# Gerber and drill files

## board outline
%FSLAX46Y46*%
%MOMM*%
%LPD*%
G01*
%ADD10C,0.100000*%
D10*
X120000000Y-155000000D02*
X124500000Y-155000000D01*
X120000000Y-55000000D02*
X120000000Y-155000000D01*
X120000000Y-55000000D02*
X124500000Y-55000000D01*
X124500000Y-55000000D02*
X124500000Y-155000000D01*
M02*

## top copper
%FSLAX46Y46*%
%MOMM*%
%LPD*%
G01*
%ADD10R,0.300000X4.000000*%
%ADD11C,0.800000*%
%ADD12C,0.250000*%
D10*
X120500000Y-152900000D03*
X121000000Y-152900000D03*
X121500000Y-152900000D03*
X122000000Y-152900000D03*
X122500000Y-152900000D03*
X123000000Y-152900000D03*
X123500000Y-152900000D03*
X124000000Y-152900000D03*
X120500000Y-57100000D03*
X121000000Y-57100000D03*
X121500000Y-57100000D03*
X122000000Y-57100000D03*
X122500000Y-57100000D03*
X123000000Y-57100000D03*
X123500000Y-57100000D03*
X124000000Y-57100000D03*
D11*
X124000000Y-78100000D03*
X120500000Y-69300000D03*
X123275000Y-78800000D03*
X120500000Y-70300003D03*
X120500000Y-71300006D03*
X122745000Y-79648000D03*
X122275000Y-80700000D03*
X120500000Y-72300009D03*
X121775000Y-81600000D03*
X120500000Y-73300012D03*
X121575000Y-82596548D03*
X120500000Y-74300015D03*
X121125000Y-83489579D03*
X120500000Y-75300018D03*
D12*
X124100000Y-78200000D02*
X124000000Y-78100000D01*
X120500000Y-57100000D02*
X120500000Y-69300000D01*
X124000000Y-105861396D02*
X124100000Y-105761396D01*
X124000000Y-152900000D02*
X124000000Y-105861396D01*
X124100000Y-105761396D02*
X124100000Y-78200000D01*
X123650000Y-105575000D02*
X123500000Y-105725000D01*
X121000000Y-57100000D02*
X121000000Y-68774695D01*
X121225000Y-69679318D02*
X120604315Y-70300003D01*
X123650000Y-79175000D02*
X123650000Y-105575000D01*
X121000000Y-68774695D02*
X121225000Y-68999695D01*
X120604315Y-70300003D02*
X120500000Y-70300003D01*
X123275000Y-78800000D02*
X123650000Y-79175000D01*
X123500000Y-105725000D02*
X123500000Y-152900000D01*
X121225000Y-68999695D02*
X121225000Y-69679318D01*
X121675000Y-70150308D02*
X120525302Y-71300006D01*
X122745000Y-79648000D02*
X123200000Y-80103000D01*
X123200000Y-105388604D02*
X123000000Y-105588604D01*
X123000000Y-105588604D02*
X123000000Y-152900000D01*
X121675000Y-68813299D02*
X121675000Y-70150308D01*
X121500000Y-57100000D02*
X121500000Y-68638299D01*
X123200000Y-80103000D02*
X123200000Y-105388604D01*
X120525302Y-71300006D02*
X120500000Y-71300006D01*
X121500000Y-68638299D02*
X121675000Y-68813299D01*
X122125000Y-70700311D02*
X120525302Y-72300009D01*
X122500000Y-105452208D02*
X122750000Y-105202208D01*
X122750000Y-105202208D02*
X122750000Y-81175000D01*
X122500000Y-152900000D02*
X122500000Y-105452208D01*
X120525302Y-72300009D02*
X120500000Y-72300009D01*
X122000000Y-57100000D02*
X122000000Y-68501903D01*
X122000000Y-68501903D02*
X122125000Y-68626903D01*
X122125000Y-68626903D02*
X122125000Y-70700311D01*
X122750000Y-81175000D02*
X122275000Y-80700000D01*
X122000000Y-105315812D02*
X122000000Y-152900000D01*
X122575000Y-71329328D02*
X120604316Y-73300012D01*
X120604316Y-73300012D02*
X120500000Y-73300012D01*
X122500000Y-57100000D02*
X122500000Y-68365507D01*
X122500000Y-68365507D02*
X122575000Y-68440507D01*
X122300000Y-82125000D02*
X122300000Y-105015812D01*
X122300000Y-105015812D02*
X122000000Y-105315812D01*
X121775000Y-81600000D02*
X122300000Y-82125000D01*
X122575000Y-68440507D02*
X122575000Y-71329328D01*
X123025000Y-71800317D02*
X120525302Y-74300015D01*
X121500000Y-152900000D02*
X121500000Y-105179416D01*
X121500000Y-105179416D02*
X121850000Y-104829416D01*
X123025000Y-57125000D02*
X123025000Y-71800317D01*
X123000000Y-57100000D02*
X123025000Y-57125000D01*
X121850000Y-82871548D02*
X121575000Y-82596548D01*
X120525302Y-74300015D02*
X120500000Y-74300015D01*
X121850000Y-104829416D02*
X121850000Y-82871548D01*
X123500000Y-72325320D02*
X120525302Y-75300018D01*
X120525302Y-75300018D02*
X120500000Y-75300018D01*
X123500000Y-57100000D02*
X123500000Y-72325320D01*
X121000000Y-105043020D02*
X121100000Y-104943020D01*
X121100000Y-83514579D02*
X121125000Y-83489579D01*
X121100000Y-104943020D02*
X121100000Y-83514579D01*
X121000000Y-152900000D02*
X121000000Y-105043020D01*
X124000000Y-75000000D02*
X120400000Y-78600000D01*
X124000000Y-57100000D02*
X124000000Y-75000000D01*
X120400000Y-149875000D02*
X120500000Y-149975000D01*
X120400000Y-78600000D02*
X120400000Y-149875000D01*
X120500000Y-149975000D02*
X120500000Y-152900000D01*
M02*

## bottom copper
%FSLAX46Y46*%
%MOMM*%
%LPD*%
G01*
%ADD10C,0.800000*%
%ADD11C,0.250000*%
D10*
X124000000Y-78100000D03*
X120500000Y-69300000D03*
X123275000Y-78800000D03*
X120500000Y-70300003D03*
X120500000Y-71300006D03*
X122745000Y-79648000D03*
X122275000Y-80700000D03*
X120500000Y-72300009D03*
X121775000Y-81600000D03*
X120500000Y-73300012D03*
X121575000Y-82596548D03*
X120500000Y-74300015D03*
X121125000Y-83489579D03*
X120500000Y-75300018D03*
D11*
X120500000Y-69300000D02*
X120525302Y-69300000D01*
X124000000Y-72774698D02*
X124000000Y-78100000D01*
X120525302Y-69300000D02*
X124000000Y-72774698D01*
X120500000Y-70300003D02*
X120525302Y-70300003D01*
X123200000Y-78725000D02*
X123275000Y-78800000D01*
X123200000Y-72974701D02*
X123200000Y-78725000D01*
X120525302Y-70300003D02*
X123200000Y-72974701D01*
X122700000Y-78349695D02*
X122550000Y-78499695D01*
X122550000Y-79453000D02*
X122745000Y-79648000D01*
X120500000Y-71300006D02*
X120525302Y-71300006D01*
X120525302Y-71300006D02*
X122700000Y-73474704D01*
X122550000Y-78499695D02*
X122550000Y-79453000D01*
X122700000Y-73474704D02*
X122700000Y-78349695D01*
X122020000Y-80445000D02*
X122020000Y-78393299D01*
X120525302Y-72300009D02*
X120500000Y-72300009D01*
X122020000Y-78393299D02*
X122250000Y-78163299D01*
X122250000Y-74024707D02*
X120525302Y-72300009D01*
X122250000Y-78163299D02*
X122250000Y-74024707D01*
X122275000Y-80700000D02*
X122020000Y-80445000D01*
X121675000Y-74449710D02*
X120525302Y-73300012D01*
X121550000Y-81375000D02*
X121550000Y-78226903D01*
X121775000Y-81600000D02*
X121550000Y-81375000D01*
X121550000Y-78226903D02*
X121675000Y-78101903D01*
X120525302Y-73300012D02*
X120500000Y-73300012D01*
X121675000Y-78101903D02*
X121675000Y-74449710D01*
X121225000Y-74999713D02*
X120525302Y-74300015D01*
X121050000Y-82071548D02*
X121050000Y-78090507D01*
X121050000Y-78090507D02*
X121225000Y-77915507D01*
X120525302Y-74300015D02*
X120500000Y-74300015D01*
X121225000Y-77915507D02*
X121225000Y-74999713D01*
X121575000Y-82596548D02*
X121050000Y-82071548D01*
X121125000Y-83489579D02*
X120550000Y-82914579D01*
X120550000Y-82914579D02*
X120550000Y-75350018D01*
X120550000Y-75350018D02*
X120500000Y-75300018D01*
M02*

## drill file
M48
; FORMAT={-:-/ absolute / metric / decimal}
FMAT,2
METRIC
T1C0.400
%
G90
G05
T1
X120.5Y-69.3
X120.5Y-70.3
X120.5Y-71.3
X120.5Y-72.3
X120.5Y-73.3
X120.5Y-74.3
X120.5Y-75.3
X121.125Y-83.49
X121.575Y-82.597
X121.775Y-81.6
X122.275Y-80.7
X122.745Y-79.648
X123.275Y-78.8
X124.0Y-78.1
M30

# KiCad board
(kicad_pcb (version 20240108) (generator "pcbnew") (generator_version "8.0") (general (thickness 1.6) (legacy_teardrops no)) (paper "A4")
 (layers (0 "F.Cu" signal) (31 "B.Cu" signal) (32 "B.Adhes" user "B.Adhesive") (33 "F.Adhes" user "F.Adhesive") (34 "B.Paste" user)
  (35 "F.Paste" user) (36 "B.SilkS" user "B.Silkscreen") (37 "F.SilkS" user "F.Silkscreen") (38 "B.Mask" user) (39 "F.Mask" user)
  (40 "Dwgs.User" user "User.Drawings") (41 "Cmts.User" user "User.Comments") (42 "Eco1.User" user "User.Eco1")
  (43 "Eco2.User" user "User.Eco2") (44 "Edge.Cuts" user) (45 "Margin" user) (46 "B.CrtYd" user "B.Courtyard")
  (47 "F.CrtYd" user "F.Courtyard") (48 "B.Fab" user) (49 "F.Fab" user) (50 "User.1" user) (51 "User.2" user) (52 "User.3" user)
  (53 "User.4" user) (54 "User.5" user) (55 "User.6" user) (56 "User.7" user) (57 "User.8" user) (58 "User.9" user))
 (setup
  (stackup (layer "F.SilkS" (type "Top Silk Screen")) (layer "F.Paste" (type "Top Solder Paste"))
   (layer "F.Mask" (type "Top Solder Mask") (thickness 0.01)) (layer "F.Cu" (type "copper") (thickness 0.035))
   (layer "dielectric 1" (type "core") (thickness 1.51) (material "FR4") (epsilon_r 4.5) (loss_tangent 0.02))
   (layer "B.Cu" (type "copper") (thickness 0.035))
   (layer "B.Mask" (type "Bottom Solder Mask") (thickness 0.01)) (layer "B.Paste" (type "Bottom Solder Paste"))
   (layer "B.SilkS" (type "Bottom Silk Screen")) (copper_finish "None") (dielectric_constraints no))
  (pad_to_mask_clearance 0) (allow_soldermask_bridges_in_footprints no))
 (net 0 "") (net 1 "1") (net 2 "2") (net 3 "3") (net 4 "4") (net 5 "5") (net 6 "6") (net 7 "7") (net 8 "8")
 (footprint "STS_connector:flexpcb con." (layer "F.Cu") (at 120 154.9)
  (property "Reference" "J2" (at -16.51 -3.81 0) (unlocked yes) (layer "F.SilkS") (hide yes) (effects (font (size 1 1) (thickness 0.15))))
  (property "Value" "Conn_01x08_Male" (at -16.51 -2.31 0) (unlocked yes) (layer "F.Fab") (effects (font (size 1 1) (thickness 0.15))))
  (pad "1" smd rect (at 0.5 -2) (size 0.3 4) (layers "F.Cu" "F.Paste" "F.Mask") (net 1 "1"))
  (pad "2" smd rect (at 1 -2) (size 0.3 4) (layers "F.Cu" "F.Paste" "F.Mask") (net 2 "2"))
  (pad "3" smd rect (at 1.5 -2) (size 0.3 4) (layers "F.Cu" "F.Paste" "F.Mask") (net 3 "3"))
  (pad "4" smd rect (at 2 -2) (size 0.3 4) (layers "F.Cu" "F.Paste" "F.Mask") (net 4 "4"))
  (pad "5" smd rect (at 2.5 -2) (size 0.3 4) (layers "F.Cu" "F.Paste" "F.Mask") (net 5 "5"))
  (pad "6" smd rect (at 3 -2) (size 0.3 4) (layers "F.Cu" "F.Paste" "F.Mask") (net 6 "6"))
  (pad "7" smd rect (at 3.5 -2) (size 0.3 4) (layers "F.Cu" "F.Paste" "F.Mask") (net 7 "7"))
  (pad "8" smd rect (at 4 -2) (size 0.3 4) (layers "F.Cu" "F.Paste" "F.Mask") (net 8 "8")))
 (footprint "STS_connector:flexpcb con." (layer "F.Cu") (at 120 59.1)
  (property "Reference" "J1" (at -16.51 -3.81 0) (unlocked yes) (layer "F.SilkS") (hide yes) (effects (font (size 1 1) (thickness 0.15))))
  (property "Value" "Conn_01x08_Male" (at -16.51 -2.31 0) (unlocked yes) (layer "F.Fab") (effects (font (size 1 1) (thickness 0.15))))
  (pad "1" smd rect (at 0.5 -2) (size 0.3 4) (layers "F.Cu" "F.Paste" "F.Mask") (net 8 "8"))
  (pad "2" smd rect (at 1 -2) (size 0.3 4) (layers "F.Cu" "F.Paste" "F.Mask") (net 7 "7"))
  (pad "3" smd rect (at 1.5 -2) (size 0.3 4) (layers "F.Cu" "F.Paste" "F.Mask") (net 6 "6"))
  (pad "4" smd rect (at 2 -2) (size 0.3 4) (layers "F.Cu" "F.Paste" "F.Mask") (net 5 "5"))
  (pad "5" smd rect (at 2.5 -2) (size 0.3 4) (layers "F.Cu" "F.Paste" "F.Mask") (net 4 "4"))
  (pad "6" smd rect (at 3 -2) (size 0.3 4) (layers "F.Cu" "F.Paste" "F.Mask") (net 3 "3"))
  (pad "7" smd rect (at 3.5 -2) (size 0.3 4) (layers "F.Cu" "F.Paste" "F.Mask") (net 2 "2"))
  (pad "8" smd rect (at 4 -2) (size 0.3 4) (layers "F.Cu" "F.Paste" "F.Mask") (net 1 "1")))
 (gr_line (start 120 155) (end 124.5 155) (stroke (width 0.1) (type solid)) (layer "Edge.Cuts"))
 (gr_line (start 120 55) (end 120 155) (stroke (width 0.1) (type solid)) (layer "Edge.Cuts"))
 (gr_line (start 120 55) (end 124.5 55) (stroke (width 0.1) (type solid)) (layer "Edge.Cuts"))
 (gr_line (start 124.5 55) (end 124.5 155) (stroke (width 0.1) (type solid)) (layer "Edge.Cuts"))
 (segment (start 124.1 78.2) (end 124 78.1) (width 0.25) (layer "F.Cu") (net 8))
 (segment (start 120.5 57.1) (end 120.5 69.3) (width 0.25) (layer "F.Cu") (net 8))
 (segment (start 124 105.861396) (end 124.1 105.761396) (width 0.25) (layer "F.Cu") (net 8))
 (segment (start 124 152.9) (end 124 105.861396) (width 0.25) (layer "F.Cu") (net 8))
 (segment (start 124.1 105.761396) (end 124.1 78.2) (width 0.25) (layer "F.Cu") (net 8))
 (via (at 124 78.1) (size 0.8) (drill 0.4) (layers "F.Cu" "B.Cu") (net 8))
 (via (at 120.5 69.3) (size 0.8) (drill 0.4) (layers "F.Cu" "B.Cu") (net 8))
 (segment (start 120.5 69.3) (end 120.525302 69.3) (width 0.25) (layer "B.Cu") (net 8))
 (segment (start 124 72.774698) (end 124 78.1) (width 0.25) (layer "B.Cu") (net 8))
 (segment (start 120.525302 69.3) (end 124 72.774698) (width 0.25) (layer "B.Cu") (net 8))
 (segment (start 123.65 105.575) (end 123.5 105.725) (width 0.25) (layer "F.Cu") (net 7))
 (segment (start 121 57.1) (end 121 68.774695) (width 0.25) (layer "F.Cu") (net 7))
 (segment (start 121.225 69.679318) (end 120.604315 70.300003) (width 0.25) (layer "F.Cu") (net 7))
 (segment (start 123.65 79.175) (end 123.65 105.575) (width 0.25) (layer "F.Cu") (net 7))
 (segment (start 121 68.774695) (end 121.225 68.999695) (width 0.25) (layer "F.Cu") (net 7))
 (segment (start 120.604315 70.300003) (end 120.5 70.300003) (width 0.25) (layer "F.Cu") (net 7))
 (segment (start 123.275 78.8) (end 123.65 79.175) (width 0.25) (layer "F.Cu") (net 7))
 (segment (start 123.5 105.725) (end 123.5 152.9) (width 0.25) (layer "F.Cu") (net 7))
 (segment (start 121.225 68.999695) (end 121.225 69.679318) (width 0.25) (layer "F.Cu") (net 7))
 (via (at 123.275 78.8) (size 0.8) (drill 0.4) (layers "F.Cu" "B.Cu") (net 7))
 (via (at 120.5 70.300003) (size 0.8) (drill 0.4) (layers "F.Cu" "B.Cu") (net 7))
 (segment (start 120.5 70.300003) (end 120.525302 70.300003) (width 0.25) (layer "B.Cu") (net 7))
 (segment (start 123.2 78.725) (end 123.275 78.8) (width 0.25) (layer "B.Cu") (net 7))
 (segment (start 123.2 72.974701) (end 123.2 78.725) (width 0.25) (layer "B.Cu") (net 7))
 (segment (start 120.525302 70.300003) (end 123.2 72.974701) (width 0.25) (layer "B.Cu") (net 7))
 (segment (start 121.675 70.150308) (end 120.525302 71.300006) (width 0.25) (layer "F.Cu") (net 6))
 (segment (start 122.745 79.648) (end 123.2 80.103) (width 0.25) (layer "F.Cu") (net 6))
 (segment (start 123.2 105.388604) (end 123 105.588604) (width 0.25) (layer "F.Cu") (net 6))
 (segment (start 123 105.588604) (end 123 152.9) (width 0.25) (layer "F.Cu") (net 6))
 (segment (start 121.675 68.813299) (end 121.675 70.150308) (width 0.25) (layer "F.Cu") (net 6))
 (segment (start 121.5 57.1) (end 121.5 68.638299) (width 0.25) (layer "F.Cu") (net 6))
 (segment (start 123.2 80.103) (end 123.2 105.388604) (width 0.25) (layer "F.Cu") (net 6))
 (segment (start 120.525302 71.300006) (end 120.5 71.300006) (width 0.25) (layer "F.Cu") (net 6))
 (segment (start 121.5 68.638299) (end 121.675 68.813299) (width 0.25) (layer "F.Cu") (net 6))
 (via (at 120.5 71.300006) (size 0.8) (drill 0.4) (layers "F.Cu" "B.Cu") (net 6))
 (via (at 122.745 79.648) (size 0.8) (drill 0.4) (layers "F.Cu" "B.Cu") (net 6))
 (segment (start 122.7 78.349695) (end 122.55 78.499695) (width 0.25) (layer "B.Cu") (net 6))
 (segment (start 122.55 79.453) (end 122.745 79.648) (width 0.25) (layer "B.Cu") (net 6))
 (segment (start 120.5 71.300006) (end 120.525302 71.300006) (width 0.25) (layer "B.Cu") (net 6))
 (segment (start 120.525302 71.300006) (end 122.7 73.474704) (width 0.25) (layer "B.Cu") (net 6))
 (segment (start 122.55 78.499695) (end 122.55 79.453) (width 0.25) (layer "B.Cu") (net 6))
 (segment (start 122.7 73.474704) (end 122.7 78.349695) (width 0.25) (layer "B.Cu") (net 6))
 (segment (start 122.125 70.700311) (end 120.525302 72.300009) (width 0.25) (layer "F.Cu") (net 5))
 (segment (start 122.5 105.452208) (end 122.75 105.202208) (width 0.25) (layer "F.Cu") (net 5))
 (segment (start 122.75 105.202208) (end 122.75 81.175) (width 0.25) (layer "F.Cu") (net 5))
 (segment (start 122.5 152.9) (end 122.5 105.452208) (width 0.25) (layer "F.Cu") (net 5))
 (segment (start 120.525302 72.300009) (end 120.5 72.300009) (width 0.25) (layer "F.Cu") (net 5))
 (segment (start 122 57.1) (end 122 68.501903) (width 0.25) (layer "F.Cu") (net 5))
 (segment (start 122 68.501903) (end 122.125 68.626903) (width 0.25) (layer "F.Cu") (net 5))
 (segment (start 122.125 68.626903) (end 122.125 70.700311) (width 0.25) (layer "F.Cu") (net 5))
 (segment (start 122.75 81.175) (end 122.275 80.7) (width 0.25) (layer "F.Cu") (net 5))
 (via (at 122.275 80.7) (size 0.8) (drill 0.4) (layers "F.Cu" "B.Cu") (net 5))
 (via (at 120.5 72.300009) (size 0.8) (drill 0.4) (layers "F.Cu" "B.Cu") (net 5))
 (segment (start 122.02 80.445) (end 122.02 78.393299) (width 0.25) (layer "B.Cu") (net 5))
 (segment (start 120.525302 72.300009) (end 120.5 72.300009) (width 0.25) (layer "B.Cu") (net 5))
 (segment (start 122.02 78.393299) (end 122.25 78.163299) (width 0.25) (layer "B.Cu") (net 5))
 (segment (start 122.25 74.024707) (end 120.525302 72.300009) (width 0.25) (layer "B.Cu") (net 5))
 (segment (start 122.25 78.163299) (end 122.25 74.024707) (width 0.25) (layer "B.Cu") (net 5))
 (segment (start 122.275 80.7) (end 122.02 80.445) (width 0.25) (layer "B.Cu") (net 5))
 (segment (start 122 105.315812) (end 122 152.9) (width 0.25) (layer "F.Cu") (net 4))
 (segment (start 122.575 71.329328) (end 120.604316 73.300012) (width 0.25) (layer "F.Cu") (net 4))
 (segment (start 120.604316 73.300012) (end 120.5 73.300012) (width 0.25) (layer "F.Cu") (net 4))
 (segment (start 122.5 57.1) (end 122.5 68.365507) (width 0.25) (layer "F.Cu") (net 4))
 (segment (start 122.5 68.365507) (end 122.575 68.440507) (width 0.25) (layer "F.Cu") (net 4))
 (segment (start 122.3 82.125) (end 122.3 105.015812) (width 0.25) (layer "F.Cu") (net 4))
 (segment (start 122.3 105.015812) (end 122 105.315812) (width 0.25) (layer "F.Cu") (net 4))
 (segment (start 121.775 81.6) (end 122.3 82.125) (width 0.25) (layer "F.Cu") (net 4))
 (segment (start 122.575 68.440507) (end 122.575 71.329328) (width 0.25) (layer "F.Cu") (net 4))
 (via (at 121.775 81.6) (size 0.8) (drill 0.4) (layers "F.Cu" "B.Cu") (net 4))
 (via (at 120.5 73.300012) (size 0.8) (drill 0.4) (layers "F.Cu" "B.Cu") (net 4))
 (segment (start 121.675 74.44971) (end 120.525302 73.300012) (width 0.25) (layer "B.Cu") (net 4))
 (segment (start 121.55 81.375) (end 121.55 78.226903) (width 0.25) (layer "B.Cu") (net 4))
 (segment (start 121.775 81.6) (end 121.55 81.375) (width 0.25) (layer "B.Cu") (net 4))
 (segment (start 121.55 78.226903) (end 121.675 78.101903) (width 0.25) (layer "B.Cu") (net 4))
 (segment (start 120.525302 73.300012) (end 120.5 73.300012) (width 0.25) (layer "B.Cu") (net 4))
 (segment (start 121.675 78.101903) (end 121.675 74.44971) (width 0.25) (layer "B.Cu") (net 4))
 (segment (start 123.025 71.800317) (end 120.525302 74.300015) (width 0.25) (layer "F.Cu") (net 3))
 (segment (start 121.5 152.9) (end 121.5 105.179416) (width 0.25) (layer "F.Cu") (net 3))
 (segment (start 121.5 105.179416) (end 121.85 104.829416) (width 0.25) (layer "F.Cu") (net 3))
 (segment (start 123.025 57.125) (end 123.025 71.800317) (width 0.25) (layer "F.Cu") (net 3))
 (segment (start 123 57.1) (end 123.025 57.125) (width 0.25) (layer "F.Cu") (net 3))
 (segment (start 121.85 82.871548) (end 121.575 82.596548) (width 0.25) (layer "F.Cu") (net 3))
 (segment (start 120.525302 74.300015) (end 120.5 74.300015) (width 0.25) (layer "F.Cu") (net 3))
 (segment (start 121.85 104.829416) (end 121.85 82.871548) (width 0.25) (layer "F.Cu") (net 3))
 (via (at 121.575 82.596548) (size 0.8) (drill 0.4) (layers "F.Cu" "B.Cu") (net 3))
 (via (at 120.5 74.300015) (size 0.8) (drill 0.4) (layers "F.Cu" "B.Cu") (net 3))
 (segment (start 121.225 74.999713) (end 120.525302 74.300015) (width 0.25) (layer "B.Cu") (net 3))
 (segment (start 121.05 82.071548) (end 121.05 78.090507) (width 0.25) (layer "B.Cu") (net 3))
 (segment (start 121.05 78.090507) (end 121.225 77.915507) (width 0.25) (layer "B.Cu") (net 3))
 (segment (start 120.525302 74.300015) (end 120.5 74.300015) (width 0.25) (layer "B.Cu") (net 3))
 (segment (start 121.225 77.915507) (end 121.225 74.999713) (width 0.25) (layer "B.Cu") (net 3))
 (segment (start 121.575 82.596548) (end 121.05 82.071548) (width 0.25) (layer "B.Cu") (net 3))
 (segment (start 123.5 72.32532) (end 120.525302 75.300018) (width 0.25) (layer "F.Cu") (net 2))
 (segment (start 120.525302 75.300018) (end 120.5 75.300018) (width 0.25) (layer "F.Cu") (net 2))
 (segment (start 123.5 57.1) (end 123.5 72.32532) (width 0.25) (layer "F.Cu") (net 2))
 (segment (start 121 105.04302) (end 121.1 104.94302) (width 0.25) (layer "F.Cu") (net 2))
 (segment (start 121.1 83.514579) (end 121.125 83.489579) (width 0.25) (layer "F.Cu") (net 2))
 (segment (start 121.1 104.94302) (end 121.1 83.514579) (width 0.25) (layer "F.Cu") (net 2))
 (segment (start 121 152.9) (end 121 105.04302) (width 0.25) (layer "F.Cu") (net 2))
 (via (at 121.125 83.489579) (size 0.8) (drill 0.4) (layers "F.Cu" "B.Cu") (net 2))
 (via (at 120.5 75.300018) (size 0.8) (drill 0.4) (layers "F.Cu" "B.Cu") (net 2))
 (segment (start 121.125 83.489579) (end 120.55 82.914579) (width 0.25) (layer "B.Cu") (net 2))
 (segment (start 120.55 82.914579) (end 120.55 75.350018) (width 0.25) (layer "B.Cu") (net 2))
 (segment (start 120.55 75.350018) (end 120.5 75.300018) (width 0.25) (layer "B.Cu") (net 2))
 (segment (start 124 75) (end 120.4 78.6) (width 0.25) (layer "F.Cu") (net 1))
 (segment (start 124 57.1) (end 124 75) (width 0.25) (layer "F.Cu") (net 1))
 (segment (start 120.4 149.875) (end 120.5 149.975) (width 0.25) (layer "F.Cu") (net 1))
 (segment (start 120.4 78.6) (end 120.4 149.875) (width 0.25) (layer "F.Cu") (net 1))
 (segment (start 120.5 149.975) (end 120.5 152.9) (width 0.25) (layer "F.Cu") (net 1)))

